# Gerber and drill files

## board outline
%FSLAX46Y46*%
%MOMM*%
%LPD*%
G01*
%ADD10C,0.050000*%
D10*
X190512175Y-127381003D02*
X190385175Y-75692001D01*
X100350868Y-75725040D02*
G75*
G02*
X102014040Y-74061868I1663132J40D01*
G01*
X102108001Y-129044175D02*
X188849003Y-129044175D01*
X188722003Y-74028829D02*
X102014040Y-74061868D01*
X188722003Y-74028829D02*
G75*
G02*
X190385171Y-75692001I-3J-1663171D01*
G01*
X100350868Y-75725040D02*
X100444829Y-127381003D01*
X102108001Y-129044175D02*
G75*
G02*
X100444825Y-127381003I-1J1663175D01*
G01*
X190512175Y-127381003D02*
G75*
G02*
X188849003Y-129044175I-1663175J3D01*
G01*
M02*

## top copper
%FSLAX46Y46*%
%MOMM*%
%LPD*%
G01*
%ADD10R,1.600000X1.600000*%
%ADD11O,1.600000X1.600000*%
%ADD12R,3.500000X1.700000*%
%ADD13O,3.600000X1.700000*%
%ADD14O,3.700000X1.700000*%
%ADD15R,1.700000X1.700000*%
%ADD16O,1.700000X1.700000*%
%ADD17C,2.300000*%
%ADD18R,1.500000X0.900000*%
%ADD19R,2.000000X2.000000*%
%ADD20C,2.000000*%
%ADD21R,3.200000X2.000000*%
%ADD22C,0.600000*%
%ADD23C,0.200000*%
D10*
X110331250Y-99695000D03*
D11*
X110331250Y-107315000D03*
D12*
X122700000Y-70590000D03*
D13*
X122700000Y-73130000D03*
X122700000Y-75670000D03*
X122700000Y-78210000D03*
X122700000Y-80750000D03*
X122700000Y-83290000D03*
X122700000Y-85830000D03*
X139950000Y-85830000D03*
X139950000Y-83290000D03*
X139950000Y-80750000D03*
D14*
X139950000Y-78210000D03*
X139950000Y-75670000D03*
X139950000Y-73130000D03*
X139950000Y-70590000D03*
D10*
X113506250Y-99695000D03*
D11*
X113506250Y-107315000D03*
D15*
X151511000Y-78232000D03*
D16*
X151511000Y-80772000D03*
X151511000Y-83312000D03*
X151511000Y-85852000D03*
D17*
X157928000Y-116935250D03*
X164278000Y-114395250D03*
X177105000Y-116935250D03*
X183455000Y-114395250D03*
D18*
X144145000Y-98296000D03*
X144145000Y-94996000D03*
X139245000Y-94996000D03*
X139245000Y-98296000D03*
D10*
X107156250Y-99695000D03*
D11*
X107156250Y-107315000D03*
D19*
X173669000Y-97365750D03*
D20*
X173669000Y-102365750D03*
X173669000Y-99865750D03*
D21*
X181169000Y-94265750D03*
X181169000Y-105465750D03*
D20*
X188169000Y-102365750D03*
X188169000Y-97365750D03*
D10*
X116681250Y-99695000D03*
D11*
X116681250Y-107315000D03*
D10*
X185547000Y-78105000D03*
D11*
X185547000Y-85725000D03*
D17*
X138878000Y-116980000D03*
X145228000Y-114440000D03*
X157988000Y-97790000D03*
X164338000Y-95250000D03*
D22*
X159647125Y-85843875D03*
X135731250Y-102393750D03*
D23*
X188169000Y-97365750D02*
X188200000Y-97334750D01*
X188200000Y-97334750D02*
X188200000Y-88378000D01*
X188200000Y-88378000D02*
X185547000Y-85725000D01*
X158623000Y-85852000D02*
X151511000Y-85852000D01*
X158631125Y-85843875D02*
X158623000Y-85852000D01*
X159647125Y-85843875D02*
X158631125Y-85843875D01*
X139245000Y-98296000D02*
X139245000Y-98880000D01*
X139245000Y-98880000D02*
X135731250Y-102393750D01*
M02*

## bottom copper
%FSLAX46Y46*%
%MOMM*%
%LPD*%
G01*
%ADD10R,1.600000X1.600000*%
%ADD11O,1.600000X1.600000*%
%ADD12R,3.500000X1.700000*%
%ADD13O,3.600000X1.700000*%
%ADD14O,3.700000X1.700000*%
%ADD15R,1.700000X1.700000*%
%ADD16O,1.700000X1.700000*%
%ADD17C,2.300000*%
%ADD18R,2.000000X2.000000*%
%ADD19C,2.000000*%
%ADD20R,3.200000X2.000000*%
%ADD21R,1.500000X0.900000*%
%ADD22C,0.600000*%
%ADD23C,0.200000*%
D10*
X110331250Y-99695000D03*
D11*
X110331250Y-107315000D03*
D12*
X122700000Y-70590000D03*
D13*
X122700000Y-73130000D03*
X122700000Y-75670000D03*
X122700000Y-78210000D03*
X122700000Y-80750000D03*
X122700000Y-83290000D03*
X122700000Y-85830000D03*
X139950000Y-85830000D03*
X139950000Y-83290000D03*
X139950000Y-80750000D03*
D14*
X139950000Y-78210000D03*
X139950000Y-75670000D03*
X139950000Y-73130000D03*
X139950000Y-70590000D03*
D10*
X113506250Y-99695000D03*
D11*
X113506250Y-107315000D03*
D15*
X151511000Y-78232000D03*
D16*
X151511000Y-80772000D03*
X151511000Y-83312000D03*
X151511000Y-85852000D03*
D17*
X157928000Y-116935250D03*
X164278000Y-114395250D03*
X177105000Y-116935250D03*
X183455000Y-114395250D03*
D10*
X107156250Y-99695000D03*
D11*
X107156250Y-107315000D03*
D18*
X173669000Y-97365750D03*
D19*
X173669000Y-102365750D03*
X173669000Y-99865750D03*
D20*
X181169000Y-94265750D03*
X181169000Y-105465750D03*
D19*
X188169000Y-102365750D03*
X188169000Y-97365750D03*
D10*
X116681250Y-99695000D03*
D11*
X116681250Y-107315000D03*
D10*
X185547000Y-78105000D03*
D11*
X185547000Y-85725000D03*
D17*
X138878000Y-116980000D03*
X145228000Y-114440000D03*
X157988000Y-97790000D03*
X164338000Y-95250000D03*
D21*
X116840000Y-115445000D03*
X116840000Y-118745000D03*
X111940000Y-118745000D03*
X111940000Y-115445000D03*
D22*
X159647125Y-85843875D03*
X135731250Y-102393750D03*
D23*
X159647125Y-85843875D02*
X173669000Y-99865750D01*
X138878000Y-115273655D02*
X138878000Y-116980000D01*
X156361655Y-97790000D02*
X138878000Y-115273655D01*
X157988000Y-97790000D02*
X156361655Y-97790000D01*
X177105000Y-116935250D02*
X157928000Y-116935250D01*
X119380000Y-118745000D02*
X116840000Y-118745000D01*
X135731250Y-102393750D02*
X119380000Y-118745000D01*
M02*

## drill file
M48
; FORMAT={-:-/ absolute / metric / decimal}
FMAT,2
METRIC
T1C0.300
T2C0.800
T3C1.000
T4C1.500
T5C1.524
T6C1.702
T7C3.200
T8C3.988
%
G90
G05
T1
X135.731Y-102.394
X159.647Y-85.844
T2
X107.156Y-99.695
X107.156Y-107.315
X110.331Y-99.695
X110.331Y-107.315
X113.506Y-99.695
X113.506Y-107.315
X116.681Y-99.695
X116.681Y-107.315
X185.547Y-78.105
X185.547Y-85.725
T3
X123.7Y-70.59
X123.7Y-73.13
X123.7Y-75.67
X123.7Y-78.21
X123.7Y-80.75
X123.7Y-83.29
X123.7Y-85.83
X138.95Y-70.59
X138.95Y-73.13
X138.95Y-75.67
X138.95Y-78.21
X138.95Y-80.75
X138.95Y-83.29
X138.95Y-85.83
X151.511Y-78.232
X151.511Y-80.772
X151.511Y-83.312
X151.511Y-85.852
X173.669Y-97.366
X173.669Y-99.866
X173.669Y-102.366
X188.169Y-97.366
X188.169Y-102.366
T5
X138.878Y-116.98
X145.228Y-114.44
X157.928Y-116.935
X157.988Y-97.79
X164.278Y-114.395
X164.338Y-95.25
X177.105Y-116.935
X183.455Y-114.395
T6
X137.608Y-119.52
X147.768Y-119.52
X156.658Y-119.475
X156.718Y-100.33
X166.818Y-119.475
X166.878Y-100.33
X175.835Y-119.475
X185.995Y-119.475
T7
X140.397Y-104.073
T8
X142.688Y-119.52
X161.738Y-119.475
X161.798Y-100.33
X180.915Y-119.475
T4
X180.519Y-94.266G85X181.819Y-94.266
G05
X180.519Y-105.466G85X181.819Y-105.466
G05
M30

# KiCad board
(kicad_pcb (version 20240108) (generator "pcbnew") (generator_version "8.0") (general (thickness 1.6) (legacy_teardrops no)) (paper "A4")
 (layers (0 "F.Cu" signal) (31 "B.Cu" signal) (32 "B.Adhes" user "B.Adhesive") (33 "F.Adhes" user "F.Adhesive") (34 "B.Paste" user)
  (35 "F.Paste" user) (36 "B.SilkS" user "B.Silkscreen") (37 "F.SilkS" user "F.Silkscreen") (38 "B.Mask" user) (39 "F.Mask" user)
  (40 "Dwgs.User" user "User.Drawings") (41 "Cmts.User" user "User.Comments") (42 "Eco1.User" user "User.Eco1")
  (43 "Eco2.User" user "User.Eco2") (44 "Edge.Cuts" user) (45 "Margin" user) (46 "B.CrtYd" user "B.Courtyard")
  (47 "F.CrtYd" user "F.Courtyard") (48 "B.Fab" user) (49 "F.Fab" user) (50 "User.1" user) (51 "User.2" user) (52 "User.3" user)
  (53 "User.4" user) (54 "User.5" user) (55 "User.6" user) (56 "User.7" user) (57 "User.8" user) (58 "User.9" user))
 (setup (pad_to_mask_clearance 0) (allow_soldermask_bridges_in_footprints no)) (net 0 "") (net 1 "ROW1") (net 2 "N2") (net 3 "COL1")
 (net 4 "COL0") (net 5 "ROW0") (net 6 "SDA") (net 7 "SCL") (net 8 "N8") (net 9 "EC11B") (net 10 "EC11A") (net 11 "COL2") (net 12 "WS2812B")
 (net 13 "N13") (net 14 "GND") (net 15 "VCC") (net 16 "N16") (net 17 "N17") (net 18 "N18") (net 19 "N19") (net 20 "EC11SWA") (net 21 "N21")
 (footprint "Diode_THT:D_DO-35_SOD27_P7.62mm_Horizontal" (layer "F.Cu") (at 110.33125 99.695 -90)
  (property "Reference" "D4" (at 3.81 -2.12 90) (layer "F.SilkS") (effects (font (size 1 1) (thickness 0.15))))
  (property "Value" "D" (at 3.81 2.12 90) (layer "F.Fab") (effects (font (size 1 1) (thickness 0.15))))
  (pad "1" thru_hole rect (at 0 0 270) (size 1.6 1.6) (drill 0.8) (layers "*.Cu" "*.Mask") (remove_unused_layers no) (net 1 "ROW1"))
  (pad "2" thru_hole oval (at 7.62 0 270) (size 1.6 1.6) (drill 0.8) (layers "*.Cu" "*.Mask") (remove_unused_layers no) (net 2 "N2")))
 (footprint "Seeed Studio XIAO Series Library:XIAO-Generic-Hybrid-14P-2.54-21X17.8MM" (layer "F.Cu") (at 131.325 78.21)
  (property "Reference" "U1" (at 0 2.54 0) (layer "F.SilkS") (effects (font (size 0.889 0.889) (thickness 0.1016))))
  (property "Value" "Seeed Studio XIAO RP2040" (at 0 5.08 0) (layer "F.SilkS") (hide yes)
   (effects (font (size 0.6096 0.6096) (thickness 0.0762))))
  (pad "1" thru_hole rect (at -7.625 -7.62) (size 3.5 1.7) (drill 1 (offset -1 0)) (layers "*.Cu" "*.Mask") (remove_unused_layers no)
   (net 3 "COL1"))
  (pad "2" thru_hole oval (at -7.625 -5.08) (size 3.6 1.7) (drill 1 (offset -1 0)) (layers "*.Cu" "*.Mask") (remove_unused_layers no)
   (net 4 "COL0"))
  (pad "3" thru_hole oval (at -7.625 -2.54) (size 3.6 1.7) (drill 1 (offset -1 0)) (layers "*.Cu" "*.Mask") (remove_unused_layers no)
   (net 1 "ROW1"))
  (pad "4" thru_hole oval (at -7.625 0) (size 3.6 1.7) (drill 1 (offset -1 0)) (layers "*.Cu" "*.Mask") (remove_unused_layers no)
   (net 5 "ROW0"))
  (pad "5" thru_hole oval (at -7.625 2.54) (size 3.6 1.7) (drill 1 (offset -1 0)) (layers "*.Cu" "*.Mask") (remove_unused_layers no)
   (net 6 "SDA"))
  (pad "6" thru_hole oval (at -7.625 5.08 180) (size 3.6 1.7) (drill 1 (offset 1 0)) (layers "*.Cu" "*.Mask") (remove_unused_layers no)
   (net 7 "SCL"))
  (pad "7" thru_hole oval (at -7.625 7.62) (size 3.6 1.7) (drill 1 (offset -1 0)) (layers "*.Cu" "*.Mask") (remove_unused_layers no)
   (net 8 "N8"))
  (pad "8" thru_hole oval (at 7.625 7.62) (size 3.6 1.7) (drill 1 (offset 1 0)) (layers "*.Cu" "*.Mask") (remove_unused_layers no)
   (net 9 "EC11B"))
  (pad "9" thru_hole oval (at 7.625 5.08) (size 3.6 1.7) (drill 1 (offset 1 0)) (layers "*.Cu" "*.Mask") (remove_unused_layers no)
   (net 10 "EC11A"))
  (pad "10" thru_hole oval (at 7.625 2.54) (size 3.6 1.7) (drill 1 (offset 1 0)) (layers "*.Cu" "*.Mask") (remove_unused_layers no)
   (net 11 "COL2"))
  (pad "11" thru_hole oval (at 7.625 0) (size 3.7 1.7) (drill 1 (offset 1 0)) (layers "*.Cu" "*.Mask") (remove_unused_layers no)
   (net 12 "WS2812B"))
  (pad "12" thru_hole oval (at 7.625 -2.54) (size 3.7 1.7) (drill 1 (offset 1 0)) (layers "*.Cu" "*.Mask") (remove_unused_layers no)
   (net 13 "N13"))
  (pad "13" thru_hole oval (at 7.625 -5.08) (size 3.7 1.7) (drill 1 (offset 1 0)) (layers "*.Cu" "*.Mask") (remove_unused_layers no)
   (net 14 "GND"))
  (pad "14" thru_hole oval (at 7.625 -7.62) (size 3.7 1.7) (drill 1 (offset 1 0)) (layers "*.Cu" "*.Mask") (remove_unused_layers no)
   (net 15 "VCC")))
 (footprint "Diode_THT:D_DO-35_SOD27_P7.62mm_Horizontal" (layer "F.Cu") (at 113.50625 99.695 -90)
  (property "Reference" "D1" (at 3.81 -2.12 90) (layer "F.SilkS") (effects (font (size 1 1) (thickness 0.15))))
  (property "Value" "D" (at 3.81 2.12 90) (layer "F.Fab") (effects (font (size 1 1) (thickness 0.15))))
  (pad "1" thru_hole rect (at 0 0 270) (size 1.6 1.6) (drill 0.8) (layers "*.Cu" "*.Mask") (remove_unused_layers no) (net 5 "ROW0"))
  (pad "2" thru_hole oval (at 7.62 0 270) (size 1.6 1.6) (drill 0.8) (layers "*.Cu" "*.Mask") (remove_unused_layers no) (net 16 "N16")))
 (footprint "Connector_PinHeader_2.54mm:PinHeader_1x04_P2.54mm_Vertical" (layer "F.Cu") (at 151.511 78.232)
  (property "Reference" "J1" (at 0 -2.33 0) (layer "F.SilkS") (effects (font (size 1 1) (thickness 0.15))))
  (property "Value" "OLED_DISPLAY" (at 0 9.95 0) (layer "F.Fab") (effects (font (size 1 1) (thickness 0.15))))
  (pad "1" thru_hole rect (at 0 0) (size 1.7 1.7) (drill 1) (layers "*.Cu" "*.Mask") (remove_unused_layers no) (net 6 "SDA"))
  (pad "2" thru_hole oval (at 0 2.54) (size 1.7 1.7) (drill 1) (layers "*.Cu" "*.Mask") (remove_unused_layers no) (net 7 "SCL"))
  (pad "3" thru_hole oval (at 0 5.08) (size 1.7 1.7) (drill 1) (layers "*.Cu" "*.Mask") (remove_unused_layers no) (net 15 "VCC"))
  (pad "4" thru_hole oval (at 0 7.62) (size 1.7 1.7) (drill 1) (layers "*.Cu" "*.Mask") (remove_unused_layers no) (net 14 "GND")))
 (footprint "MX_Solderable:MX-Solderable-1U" (layer "F.Cu") (at 161.738 119.47525)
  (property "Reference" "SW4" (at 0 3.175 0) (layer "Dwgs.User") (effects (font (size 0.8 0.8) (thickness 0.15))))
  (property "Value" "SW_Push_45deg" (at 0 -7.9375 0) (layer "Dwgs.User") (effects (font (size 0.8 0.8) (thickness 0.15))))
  (pad "" np_thru_hole circle (at -5.08 0 48.099) (size 1.7018 1.7018) (drill 1.7018) (layers "F&B.Cu" "*.Mask"))
  (pad "" np_thru_hole circle (at 0 0) (size 3.9878 3.9878) (drill 3.9878) (layers "*.Cu" "*.Mask"))
  (pad "" np_thru_hole circle (at 5.08 0 48.099) (size 1.7018 1.7018) (drill 1.7018) (layers "F&B.Cu" "*.Mask"))
  (pad "1" thru_hole circle (at -3.81 -2.54) (size 2.3 2.3) (drill 1.524) (layers "*.Cu" "B.Mask") (remove_unused_layers no) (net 3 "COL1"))
  (pad "2" thru_hole circle (at 2.54 -5.08) (size 2.3 2.3) (drill 1.524) (layers "*.Cu" "B.Mask") (remove_unused_layers no) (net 2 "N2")))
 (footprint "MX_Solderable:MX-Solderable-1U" (layer "F.Cu") (at 180.915 119.47525)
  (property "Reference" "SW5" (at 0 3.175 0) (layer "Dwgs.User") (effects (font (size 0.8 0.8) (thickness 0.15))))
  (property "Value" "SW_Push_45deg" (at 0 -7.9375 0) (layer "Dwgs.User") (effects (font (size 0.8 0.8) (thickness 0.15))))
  (pad "" np_thru_hole circle (at -5.08 0 48.099) (size 1.7018 1.7018) (drill 1.7018) (layers "F&B.Cu" "*.Mask"))
  (pad "" np_thru_hole circle (at 0 0) (size 3.9878 3.9878) (drill 3.9878) (layers "*.Cu" "*.Mask"))
  (pad "" np_thru_hole circle (at 5.08 0 48.099) (size 1.7018 1.7018) (drill 1.7018) (layers "F&B.Cu" "*.Mask"))
  (pad "1" thru_hole circle (at -3.81 -2.54) (size 2.3 2.3) (drill 1.524) (layers "*.Cu" "B.Mask") (remove_unused_layers no) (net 3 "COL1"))
  (pad "2" thru_hole circle (at 2.54 -5.08) (size 2.3 2.3) (drill 1.524) (layers "*.Cu" "B.Mask") (remove_unused_layers no) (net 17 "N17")))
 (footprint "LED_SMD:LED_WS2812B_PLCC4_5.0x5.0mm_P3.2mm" (layer "F.Cu") (at 141.695 96.646 180)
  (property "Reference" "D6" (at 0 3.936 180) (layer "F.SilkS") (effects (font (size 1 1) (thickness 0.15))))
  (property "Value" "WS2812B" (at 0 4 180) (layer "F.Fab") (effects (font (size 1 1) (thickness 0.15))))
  (pad "1" smd rect (at -2.45 -1.65 180) (size 1.5 0.9) (layers "F.Cu" "F.Paste" "F.Mask") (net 15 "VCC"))
  (pad "2" smd rect (at -2.45 1.65 180) (size 1.5 0.9) (layers "F.Cu" "F.Paste" "F.Mask") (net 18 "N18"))
  (pad "3" smd rect (at 2.45 1.65 180) (size 1.5 0.9) (layers "F.Cu" "F.Paste" "F.Mask") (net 14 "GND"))
  (pad "4" smd rect (at 2.45 -1.65 180) (size 1.5 0.9) (layers "F.Cu" "F.Paste" "F.Mask") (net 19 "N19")))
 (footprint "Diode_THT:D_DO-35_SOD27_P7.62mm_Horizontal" (layer "F.Cu") (at 107.15625 99.695 -90)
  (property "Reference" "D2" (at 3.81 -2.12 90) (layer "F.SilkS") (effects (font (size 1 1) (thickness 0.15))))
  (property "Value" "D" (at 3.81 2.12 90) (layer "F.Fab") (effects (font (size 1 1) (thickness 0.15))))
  (pad "1" thru_hole rect (at 0 0 270) (size 1.6 1.6) (drill 0.8) (layers "*.Cu" "*.Mask") (remove_unused_layers no) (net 5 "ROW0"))
  (pad "2" thru_hole oval (at 7.62 0 270) (size 1.6 1.6) (drill 0.8) (layers "*.Cu" "*.Mask") (remove_unused_layers no) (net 17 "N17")))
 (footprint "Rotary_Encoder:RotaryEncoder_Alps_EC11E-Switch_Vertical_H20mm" (layer "F.Cu") (at 173.669 97.36575)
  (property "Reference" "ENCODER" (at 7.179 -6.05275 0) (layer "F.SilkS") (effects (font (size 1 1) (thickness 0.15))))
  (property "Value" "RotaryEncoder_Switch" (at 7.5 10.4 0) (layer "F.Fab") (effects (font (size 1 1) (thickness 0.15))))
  (pad "A" thru_hole rect (at 0 0) (size 2 2) (drill 1) (layers "*.Cu" "*.Mask") (remove_unused_layers no) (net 10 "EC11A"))
  (pad "B" thru_hole circle (at 0 5) (size 2 2) (drill 1) (layers "*.Cu" "*.Mask") (remove_unused_layers no) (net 9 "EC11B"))
  (pad "C" thru_hole circle (at 0 2.5) (size 2 2) (drill 1) (layers "*.Cu" "*.Mask") (remove_unused_layers no) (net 14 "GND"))
  (pad "MP" thru_hole rect (at 7.5 -3.1) (size 3.2 2) (drill oval 2.8 1.5) (layers "*.Cu" "*.Mask") (remove_unused_layers no))
  (pad "MP" thru_hole rect (at 7.5 8.1) (size 3.2 2) (drill oval 2.8 1.5) (layers "*.Cu" "*.Mask") (remove_unused_layers no))
  (pad "S1" thru_hole circle (at 14.5 5) (size 2 2) (drill 1) (layers "*.Cu" "*.Mask") (remove_unused_layers no) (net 11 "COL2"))
  (pad "S2" thru_hole circle (at 14.5 0) (size 2 2) (drill 1) (layers "*.Cu" "*.Mask") (remove_unused_layers no) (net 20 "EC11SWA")))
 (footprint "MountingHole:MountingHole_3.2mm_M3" (layer "F.Cu") (at 140.397 104.07275)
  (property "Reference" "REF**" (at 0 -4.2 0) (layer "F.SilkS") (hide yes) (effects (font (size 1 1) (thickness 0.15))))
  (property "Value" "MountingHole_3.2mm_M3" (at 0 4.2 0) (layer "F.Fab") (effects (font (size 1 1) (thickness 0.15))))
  (pad "" np_thru_hole circle (at 0 0) (size 3.2 3.2) (drill 3.2) (layers "*.Cu" "*.Mask")))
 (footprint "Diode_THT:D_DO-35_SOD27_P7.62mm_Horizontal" (layer "F.Cu") (at 116.68125 99.695 -90)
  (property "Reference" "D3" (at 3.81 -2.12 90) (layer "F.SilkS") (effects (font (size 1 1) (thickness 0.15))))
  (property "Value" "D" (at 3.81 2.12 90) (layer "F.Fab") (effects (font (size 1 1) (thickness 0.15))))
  (pad "1" thru_hole rect (at 0 0 270) (size 1.6 1.6) (drill 0.8) (layers "*.Cu" "*.Mask") (remove_unused_layers no) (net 1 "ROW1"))
  (pad "2" thru_hole oval (at 7.62 0 270) (size 1.6 1.6) (drill 0.8) (layers "*.Cu" "*.Mask") (remove_unused_layers no) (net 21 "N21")))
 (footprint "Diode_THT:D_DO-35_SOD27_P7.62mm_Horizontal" (layer "F.Cu") (at 185.547 78.105 -90)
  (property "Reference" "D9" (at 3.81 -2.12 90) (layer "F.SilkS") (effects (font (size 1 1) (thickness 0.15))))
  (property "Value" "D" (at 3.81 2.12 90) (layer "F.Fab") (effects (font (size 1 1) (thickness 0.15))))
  (pad "1" thru_hole rect (at 0 0 270) (size 1.6 1.6) (drill 0.8) (layers "*.Cu" "*.Mask") (remove_unused_layers no) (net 5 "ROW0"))
  (pad "2" thru_hole oval (at 7.62 0 270) (size 1.6 1.6) (drill 0.8) (layers "*.Cu" "*.Mask") (remove_unused_layers no) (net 20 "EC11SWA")))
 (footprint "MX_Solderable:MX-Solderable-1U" (layer "F.Cu") (at 142.688 119.52)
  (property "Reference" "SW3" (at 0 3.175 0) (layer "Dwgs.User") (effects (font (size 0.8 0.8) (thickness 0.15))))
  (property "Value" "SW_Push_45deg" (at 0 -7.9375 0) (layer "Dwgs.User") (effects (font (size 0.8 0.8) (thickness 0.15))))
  (pad "" np_thru_hole circle (at -5.08 0 48.099) (size 1.7018 1.7018) (drill 1.7018) (layers "F&B.Cu" "*.Mask"))
  (pad "" np_thru_hole circle (at 0 0) (size 3.9878 3.9878) (drill 3.9878) (layers "*.Cu" "*.Mask"))
  (pad "" np_thru_hole circle (at 5.08 0 48.099) (size 1.7018 1.7018) (drill 1.7018) (layers "F&B.Cu" "*.Mask"))
  (pad "1" thru_hole circle (at -3.81 -2.54) (size 2.3 2.3) (drill 1.524) (layers "*.Cu" "B.Mask") (remove_unused_layers no) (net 4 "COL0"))
  (pad "2" thru_hole circle (at 2.54 -5.08) (size 2.3 2.3) (drill 1.524) (layers "*.Cu" "B.Mask") (remove_unused_layers no) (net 21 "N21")))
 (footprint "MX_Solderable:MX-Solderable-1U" (layer "F.Cu") (at 161.798 100.33)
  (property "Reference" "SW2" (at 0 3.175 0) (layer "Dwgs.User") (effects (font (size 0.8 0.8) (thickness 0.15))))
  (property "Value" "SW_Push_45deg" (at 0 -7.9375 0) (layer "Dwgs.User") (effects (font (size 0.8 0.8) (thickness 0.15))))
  (pad "" np_thru_hole circle (at -5.08 0 48.099) (size 1.7018 1.7018) (drill 1.7018) (layers "F&B.Cu" "*.Mask"))
  (pad "" np_thru_hole circle (at 0 0) (size 3.9878 3.9878) (drill 3.9878) (layers "*.Cu" "*.Mask"))
  (pad "" np_thru_hole circle (at 5.08 0 48.099) (size 1.7018 1.7018) (drill 1.7018) (layers "F&B.Cu" "*.Mask"))
  (pad "1" thru_hole circle (at -3.81 -2.54) (size 2.3 2.3) (drill 1.524) (layers "*.Cu" "B.Mask") (remove_unused_layers no) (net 4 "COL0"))
  (pad "2" thru_hole circle (at 2.54 -5.08) (size 2.3 2.3) (drill 1.524) (layers "*.Cu" "B.Mask") (remove_unused_layers no) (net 16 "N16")))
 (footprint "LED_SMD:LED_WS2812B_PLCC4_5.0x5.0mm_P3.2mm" (layer "B.Cu") (at 114.39 117.095 180)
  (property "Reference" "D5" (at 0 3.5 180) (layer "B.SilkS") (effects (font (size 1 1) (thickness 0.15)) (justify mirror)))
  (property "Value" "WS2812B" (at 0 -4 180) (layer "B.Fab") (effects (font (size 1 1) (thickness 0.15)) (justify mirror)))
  (pad "1" smd rect (at -2.45 1.65 180) (size 1.5 0.9) (layers "B.Cu" "B.Paste" "B.Mask") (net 15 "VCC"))
  (pad "2" smd rect (at -2.45 -1.65 180) (size 1.5 0.9) (layers "B.Cu" "B.Paste" "B.Mask") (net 19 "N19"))
  (pad "3" smd rect (at 2.45 -1.65 180) (size 1.5 0.9) (layers "B.Cu" "B.Paste" "B.Mask") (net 14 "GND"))
  (pad "4" smd rect (at 2.45 1.65 180) (size 1.5 0.9) (layers "B.Cu" "B.Paste" "B.Mask") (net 12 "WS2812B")))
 (gr_line (start 190.512175 127.381003) (end 190.385175 75.692001) (stroke (width 0.05) (type default)) (layer "Edge.Cuts"))
 (gr_arc (start 100.350868 75.72504) (mid 100.838 74.549) (end 102.01404 74.061868) (stroke (width 0.05) (type default)) (layer "Edge.Cuts"))
 (gr_line (start 102.108001 129.044175) (end 188.849003 129.044175) (stroke (width 0.05) (type default)) (layer "Edge.Cuts"))
 (gr_line (start 188.722003 74.028829) (end 102.01404 74.061868) (stroke (width 0.05) (type default)) (layer "Edge.Cuts"))
 (gr_arc (start 188.722003 74.028829) (mid 189.898043 74.515961) (end 190.385175 75.692001) (stroke (width 0.05) (type default))
  (layer "Edge.Cuts"))
 (gr_line (start 100.350868 75.72504) (end 100.444829 127.381003) (stroke (width 0.05) (type default)) (layer "Edge.Cuts"))
 (gr_arc (start 102.108001 129.044175) (mid 100.931961 128.557043) (end 100.444829 127.381003) (stroke (width 0.05) (type default))
  (layer "Edge.Cuts"))
 (gr_arc (start 190.512175 127.381003) (mid 190.025043 128.557043) (end 188.849003 129.044175) (stroke (width 0.05) (type default))
  (layer "Edge.Cuts"))
 (segment (start 188.169 97.36575) (end 188.2 97.33475) (width 0.2) (layer "F.Cu") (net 20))
 (segment (start 188.2 97.33475) (end 188.2 88.378) (width 0.2) (layer "F.Cu") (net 20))
 (segment (start 188.2 88.378) (end 185.547 85.725) (width 0.2) (layer "F.Cu") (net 20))
 (segment (start 158.623 85.852) (end 151.511 85.852) (width 0.2) (layer "F.Cu") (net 14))
 (segment (start 158.631125 85.843875) (end 158.623 85.852) (width 0.2) (layer "F.Cu") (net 14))
 (segment (start 159.647125 85.843875) (end 158.631125 85.843875) (width 0.2) (layer "F.Cu") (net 14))
 (via (at 159.647125 85.843875) (size 0.6) (drill 0.3) (layers "F.Cu" "B.Cu") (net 14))
 (segment (start 159.647125 85.843875) (end 173.669 99.86575) (width 0.2) (layer "B.Cu") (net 14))
 (segment (start 138.878 115.273655) (end 138.878 116.98) (width 0.2) (layer "B.Cu") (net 4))
 (segment (start 156.361655 97.79) (end 138.878 115.273655) (width 0.2) (layer "B.Cu") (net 4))
 (segment (start 157.988 97.79) (end 156.361655 97.79) (width 0.2) (layer "B.Cu") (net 4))
 (segment (start 177.105 116.93525) (end 157.928 116.93525) (width 0.2) (layer "B.Cu") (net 3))
 (segment (start 139.245 98.296) (end 139.245 98.88) (width 0.2) (layer "F.Cu") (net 19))
 (segment (start 139.245 98.88) (end 135.73125 102.39375) (width 0.2) (layer "F.Cu") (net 19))
 (via (at 135.73125 102.39375) (size 0.6) (drill 0.3) (layers "F.Cu" "B.Cu") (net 19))
 (segment (start 119.38 118.745) (end 116.84 118.745) (width 0.2) (layer "B.Cu") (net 19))
 (segment (start 135.73125 102.39375) (end 119.38 118.745) (width 0.2) (layer "B.Cu") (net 19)))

